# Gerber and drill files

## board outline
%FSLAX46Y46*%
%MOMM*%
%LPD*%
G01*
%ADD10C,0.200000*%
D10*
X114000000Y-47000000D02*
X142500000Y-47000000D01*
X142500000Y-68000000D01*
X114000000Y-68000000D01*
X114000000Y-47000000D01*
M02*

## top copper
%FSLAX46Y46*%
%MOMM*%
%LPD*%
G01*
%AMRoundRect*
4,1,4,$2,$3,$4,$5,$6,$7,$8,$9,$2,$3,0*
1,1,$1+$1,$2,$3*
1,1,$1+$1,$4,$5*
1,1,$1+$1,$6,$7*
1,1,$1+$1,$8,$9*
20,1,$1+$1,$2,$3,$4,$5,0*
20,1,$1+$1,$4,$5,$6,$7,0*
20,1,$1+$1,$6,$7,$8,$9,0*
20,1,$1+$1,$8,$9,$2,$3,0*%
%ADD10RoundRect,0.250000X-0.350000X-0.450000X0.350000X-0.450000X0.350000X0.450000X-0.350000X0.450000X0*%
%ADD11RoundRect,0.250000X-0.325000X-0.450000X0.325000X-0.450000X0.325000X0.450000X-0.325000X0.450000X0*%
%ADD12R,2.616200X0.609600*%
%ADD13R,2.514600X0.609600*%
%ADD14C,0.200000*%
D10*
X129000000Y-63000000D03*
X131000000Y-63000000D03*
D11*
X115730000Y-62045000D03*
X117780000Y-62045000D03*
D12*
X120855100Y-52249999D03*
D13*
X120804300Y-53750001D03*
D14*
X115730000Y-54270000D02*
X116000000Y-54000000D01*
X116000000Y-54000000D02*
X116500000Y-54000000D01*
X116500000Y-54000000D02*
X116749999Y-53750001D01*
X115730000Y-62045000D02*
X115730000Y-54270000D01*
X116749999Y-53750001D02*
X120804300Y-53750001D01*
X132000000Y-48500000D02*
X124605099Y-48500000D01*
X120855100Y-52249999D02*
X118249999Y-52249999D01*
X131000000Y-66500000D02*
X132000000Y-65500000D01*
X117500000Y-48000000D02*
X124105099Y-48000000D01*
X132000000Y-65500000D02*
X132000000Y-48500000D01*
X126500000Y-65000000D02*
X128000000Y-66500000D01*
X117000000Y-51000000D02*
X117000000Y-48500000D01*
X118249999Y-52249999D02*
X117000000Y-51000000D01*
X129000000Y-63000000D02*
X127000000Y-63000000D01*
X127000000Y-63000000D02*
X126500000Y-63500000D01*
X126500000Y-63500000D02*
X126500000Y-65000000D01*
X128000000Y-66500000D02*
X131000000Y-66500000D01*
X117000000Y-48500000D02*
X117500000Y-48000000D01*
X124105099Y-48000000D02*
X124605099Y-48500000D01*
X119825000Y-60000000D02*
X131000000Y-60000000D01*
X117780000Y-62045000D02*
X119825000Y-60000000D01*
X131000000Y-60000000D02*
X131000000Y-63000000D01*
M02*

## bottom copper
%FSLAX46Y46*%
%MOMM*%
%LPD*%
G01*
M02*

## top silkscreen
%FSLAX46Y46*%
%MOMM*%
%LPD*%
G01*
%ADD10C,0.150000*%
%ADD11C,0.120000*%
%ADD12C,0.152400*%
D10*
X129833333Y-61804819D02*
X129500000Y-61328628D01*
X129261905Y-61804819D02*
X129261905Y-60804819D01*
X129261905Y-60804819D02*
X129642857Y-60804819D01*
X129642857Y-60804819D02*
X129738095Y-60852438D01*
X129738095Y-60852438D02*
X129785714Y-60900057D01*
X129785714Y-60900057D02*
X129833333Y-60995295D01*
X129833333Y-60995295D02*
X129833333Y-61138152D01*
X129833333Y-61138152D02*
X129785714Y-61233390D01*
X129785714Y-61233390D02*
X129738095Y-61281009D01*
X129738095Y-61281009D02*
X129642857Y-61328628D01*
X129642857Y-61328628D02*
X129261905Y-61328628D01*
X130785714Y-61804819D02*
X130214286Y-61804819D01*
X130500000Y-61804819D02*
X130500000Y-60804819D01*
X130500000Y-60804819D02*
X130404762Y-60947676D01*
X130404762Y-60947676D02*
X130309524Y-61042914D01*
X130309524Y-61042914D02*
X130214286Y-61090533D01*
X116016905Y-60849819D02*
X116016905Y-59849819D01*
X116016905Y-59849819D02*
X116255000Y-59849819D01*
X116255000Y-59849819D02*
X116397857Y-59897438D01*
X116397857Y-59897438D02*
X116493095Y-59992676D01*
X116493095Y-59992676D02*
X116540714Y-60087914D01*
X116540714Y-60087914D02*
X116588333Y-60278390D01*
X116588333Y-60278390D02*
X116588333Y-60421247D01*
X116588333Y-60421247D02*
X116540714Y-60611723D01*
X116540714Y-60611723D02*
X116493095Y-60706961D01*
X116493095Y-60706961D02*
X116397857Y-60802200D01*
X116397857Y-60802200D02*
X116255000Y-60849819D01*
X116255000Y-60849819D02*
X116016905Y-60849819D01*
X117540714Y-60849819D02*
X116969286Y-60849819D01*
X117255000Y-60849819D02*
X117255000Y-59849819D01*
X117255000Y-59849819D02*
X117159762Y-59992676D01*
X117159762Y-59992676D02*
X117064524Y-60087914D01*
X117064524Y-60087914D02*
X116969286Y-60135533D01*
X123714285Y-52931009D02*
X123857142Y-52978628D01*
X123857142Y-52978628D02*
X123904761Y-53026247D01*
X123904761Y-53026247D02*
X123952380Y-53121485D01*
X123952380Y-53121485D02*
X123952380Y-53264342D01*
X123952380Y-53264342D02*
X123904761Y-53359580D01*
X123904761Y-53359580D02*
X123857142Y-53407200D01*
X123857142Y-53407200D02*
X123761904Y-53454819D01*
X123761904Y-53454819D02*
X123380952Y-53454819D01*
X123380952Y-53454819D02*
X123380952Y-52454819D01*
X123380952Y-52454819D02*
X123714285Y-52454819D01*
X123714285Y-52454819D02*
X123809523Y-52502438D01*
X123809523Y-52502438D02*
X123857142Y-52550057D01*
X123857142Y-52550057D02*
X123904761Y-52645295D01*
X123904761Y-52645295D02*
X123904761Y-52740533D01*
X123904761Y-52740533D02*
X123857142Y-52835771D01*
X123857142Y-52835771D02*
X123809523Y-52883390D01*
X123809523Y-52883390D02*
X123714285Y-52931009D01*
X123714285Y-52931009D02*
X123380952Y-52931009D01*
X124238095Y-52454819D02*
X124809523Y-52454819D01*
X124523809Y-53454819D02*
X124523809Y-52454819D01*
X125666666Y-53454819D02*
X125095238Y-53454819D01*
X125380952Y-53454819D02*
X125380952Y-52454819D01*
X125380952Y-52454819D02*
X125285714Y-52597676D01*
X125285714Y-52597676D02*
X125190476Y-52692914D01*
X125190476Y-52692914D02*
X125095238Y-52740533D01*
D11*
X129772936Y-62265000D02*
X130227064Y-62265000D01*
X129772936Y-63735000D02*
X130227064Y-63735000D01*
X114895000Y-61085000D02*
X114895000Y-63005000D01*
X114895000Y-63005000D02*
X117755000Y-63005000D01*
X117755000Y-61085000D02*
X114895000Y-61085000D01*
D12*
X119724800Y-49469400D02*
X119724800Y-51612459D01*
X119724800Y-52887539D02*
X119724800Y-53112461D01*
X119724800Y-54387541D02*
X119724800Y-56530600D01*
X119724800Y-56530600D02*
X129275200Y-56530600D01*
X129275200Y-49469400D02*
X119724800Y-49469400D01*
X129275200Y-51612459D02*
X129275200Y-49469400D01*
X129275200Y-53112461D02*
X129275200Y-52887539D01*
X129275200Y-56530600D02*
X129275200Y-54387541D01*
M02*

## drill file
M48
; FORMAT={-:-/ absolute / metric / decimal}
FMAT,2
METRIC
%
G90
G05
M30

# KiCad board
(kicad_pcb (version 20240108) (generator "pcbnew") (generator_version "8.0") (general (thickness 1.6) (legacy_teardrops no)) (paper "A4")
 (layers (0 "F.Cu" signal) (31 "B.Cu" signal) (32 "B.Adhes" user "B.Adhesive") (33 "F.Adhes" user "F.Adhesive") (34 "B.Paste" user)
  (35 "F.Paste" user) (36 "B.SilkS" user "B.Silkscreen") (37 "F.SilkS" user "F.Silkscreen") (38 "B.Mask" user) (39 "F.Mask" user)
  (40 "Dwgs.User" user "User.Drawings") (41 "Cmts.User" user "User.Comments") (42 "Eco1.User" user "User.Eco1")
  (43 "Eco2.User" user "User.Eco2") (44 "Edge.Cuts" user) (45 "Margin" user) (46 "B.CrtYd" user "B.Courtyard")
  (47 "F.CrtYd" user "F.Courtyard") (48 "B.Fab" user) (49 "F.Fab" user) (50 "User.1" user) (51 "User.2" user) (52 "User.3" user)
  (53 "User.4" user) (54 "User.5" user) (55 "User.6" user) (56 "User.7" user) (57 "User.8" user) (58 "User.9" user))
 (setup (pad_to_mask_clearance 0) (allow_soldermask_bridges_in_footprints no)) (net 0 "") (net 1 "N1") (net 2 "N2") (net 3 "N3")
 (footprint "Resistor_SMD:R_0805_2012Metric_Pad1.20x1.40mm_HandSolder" (layer "F.Cu") (at 130 63)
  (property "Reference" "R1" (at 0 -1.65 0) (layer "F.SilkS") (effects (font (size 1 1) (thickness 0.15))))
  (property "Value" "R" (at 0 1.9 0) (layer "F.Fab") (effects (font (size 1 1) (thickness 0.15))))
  (fp_line (start -0.227064 -0.735) (end 0.227064 -0.735) (stroke (width 0.12) (type solid)) (layer "F.SilkS"))
  (fp_line (start -0.227064 0.735) (end 0.227064 0.735) (stroke (width 0.12) (type solid)) (layer "F.SilkS"))
  (pad "1" smd roundrect (at -1 0) (size 1.2 1.4) (layers "F.Cu" "F.Paste" "F.Mask") (roundrect_rratio 0.208333) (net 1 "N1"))
  (pad "2" smd roundrect (at 1 0) (size 1.2 1.4) (layers "F.Cu" "F.Paste" "F.Mask") (roundrect_rratio 0.208333) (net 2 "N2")))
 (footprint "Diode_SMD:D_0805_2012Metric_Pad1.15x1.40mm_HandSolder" (layer "F.Cu") (at 116.755 62.045)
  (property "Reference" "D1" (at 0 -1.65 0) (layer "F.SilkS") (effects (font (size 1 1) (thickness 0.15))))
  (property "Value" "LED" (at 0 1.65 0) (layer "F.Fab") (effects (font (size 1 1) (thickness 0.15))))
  (fp_line (start -1.86 -0.96) (end -1.86 0.96) (stroke (width 0.12) (type solid)) (layer "F.SilkS"))
  (fp_line (start -1.86 0.96) (end 1 0.96) (stroke (width 0.12) (type solid)) (layer "F.SilkS"))
  (fp_line (start 1 -0.96) (end -1.86 -0.96) (stroke (width 0.12) (type solid)) (layer "F.SilkS"))
  (pad "1" smd roundrect (at -1.025 0) (size 1.15 1.4) (layers "F.Cu" "F.Paste" "F.Mask") (roundrect_rratio 0.217391) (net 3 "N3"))
  (pad "2" smd roundrect (at 1.025 0) (size 1.15 1.4) (layers "F.Cu" "F.Paste" "F.Mask") (roundrect_rratio 0.217391) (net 2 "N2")))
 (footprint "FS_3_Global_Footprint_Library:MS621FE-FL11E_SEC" (layer "F.Cu") (at 124.5 53)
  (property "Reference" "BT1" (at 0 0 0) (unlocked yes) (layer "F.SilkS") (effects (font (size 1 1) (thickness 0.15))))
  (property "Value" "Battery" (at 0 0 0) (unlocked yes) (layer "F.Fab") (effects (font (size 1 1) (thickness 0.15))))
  (fp_line (start -4.7752 -3.5306) (end -4.7752 -1.387541) (stroke (width 0.1524) (type solid)) (layer "F.SilkS"))
  (fp_line (start -4.7752 -0.112461) (end -4.7752 0.112461) (stroke (width 0.1524) (type solid)) (layer "F.SilkS"))
  (fp_line (start -4.7752 1.387541) (end -4.7752 3.5306) (stroke (width 0.1524) (type solid)) (layer "F.SilkS"))
  (fp_line (start -4.7752 3.5306) (end 4.7752 3.5306) (stroke (width 0.1524) (type solid)) (layer "F.SilkS"))
  (fp_line (start 4.7752 -3.5306) (end -4.7752 -3.5306) (stroke (width 0.1524) (type solid)) (layer "F.SilkS"))
  (fp_line (start 4.7752 -1.387541) (end 4.7752 -3.5306) (stroke (width 0.1524) (type solid)) (layer "F.SilkS"))
  (fp_line (start 4.7752 0.112461) (end 4.7752 -0.112461) (stroke (width 0.1524) (type solid)) (layer "F.SilkS"))
  (fp_line (start 4.7752 3.5306) (end 4.7752 1.387541) (stroke (width 0.1524) (type solid)) (layer "F.SilkS"))
  (pad "1" smd rect (at -3.6449 -0.750001) (size 2.6162 0.6096) (layers "F.Cu" "F.Paste" "F.Mask") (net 1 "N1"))
  (pad "2" smd rect (at -3.6957 0.750001) (size 2.5146 0.6096) (layers "F.Cu" "F.Paste" "F.Mask") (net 3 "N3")))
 (gr_rect (start 114 47) (end 142.5 68) (stroke (width 0.2) (type default)) (fill none) (layer "Edge.Cuts"))
 (segment (start 115.73 54.27) (end 116 54) (width 0.2) (layer "F.Cu") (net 3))
 (segment (start 116 54) (end 116.5 54) (width 0.2) (layer "F.Cu") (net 3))
 (segment (start 116.5 54) (end 116.749999 53.750001) (width 0.2) (layer "F.Cu") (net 3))
 (segment (start 115.73 62.045) (end 115.73 54.27) (width 0.2) (layer "F.Cu") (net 3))
 (segment (start 116.749999 53.750001) (end 120.8043 53.750001) (width 0.2) (layer "F.Cu") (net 3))
 (segment (start 132 48.5) (end 124.605099 48.5) (width 0.2) (layer "F.Cu") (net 1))
 (segment (start 120.8551 52.249999) (end 118.249999 52.249999) (width 0.2) (layer "F.Cu") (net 1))
 (segment (start 131 66.5) (end 132 65.5) (width 0.2) (layer "F.Cu") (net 1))
 (segment (start 117.5 48) (end 124.105099 48) (width 0.2) (layer "F.Cu") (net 1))
 (segment (start 132 65.5) (end 132 48.5) (width 0.2) (layer "F.Cu") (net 1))
 (segment (start 126.5 65) (end 128 66.5) (width 0.2) (layer "F.Cu") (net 1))
 (segment (start 117 51) (end 117 48.5) (width 0.2) (layer "F.Cu") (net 1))
 (segment (start 118.249999 52.249999) (end 117 51) (width 0.2) (layer "F.Cu") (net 1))
 (segment (start 129 63) (end 127 63) (width 0.2) (layer "F.Cu") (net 1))
 (segment (start 127 63) (end 126.5 63.5) (width 0.2) (layer "F.Cu") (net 1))
 (segment (start 126.5 63.5) (end 126.5 65) (width 0.2) (layer "F.Cu") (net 1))
 (segment (start 128 66.5) (end 131 66.5) (width 0.2) (layer "F.Cu") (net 1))
 (segment (start 117 48.5) (end 117.5 48) (width 0.2) (layer "F.Cu") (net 1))
 (segment (start 124.105099 48) (end 124.605099 48.5) (width 0.2) (layer "F.Cu") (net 1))
 (segment (start 119.825 60) (end 131 60) (width 0.2) (layer "F.Cu") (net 2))
 (segment (start 117.78 62.045) (end 119.825 60) (width 0.2) (layer "F.Cu") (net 2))
 (segment (start 131 60) (end 131 63) (width 0.2) (layer "F.Cu") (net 2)))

